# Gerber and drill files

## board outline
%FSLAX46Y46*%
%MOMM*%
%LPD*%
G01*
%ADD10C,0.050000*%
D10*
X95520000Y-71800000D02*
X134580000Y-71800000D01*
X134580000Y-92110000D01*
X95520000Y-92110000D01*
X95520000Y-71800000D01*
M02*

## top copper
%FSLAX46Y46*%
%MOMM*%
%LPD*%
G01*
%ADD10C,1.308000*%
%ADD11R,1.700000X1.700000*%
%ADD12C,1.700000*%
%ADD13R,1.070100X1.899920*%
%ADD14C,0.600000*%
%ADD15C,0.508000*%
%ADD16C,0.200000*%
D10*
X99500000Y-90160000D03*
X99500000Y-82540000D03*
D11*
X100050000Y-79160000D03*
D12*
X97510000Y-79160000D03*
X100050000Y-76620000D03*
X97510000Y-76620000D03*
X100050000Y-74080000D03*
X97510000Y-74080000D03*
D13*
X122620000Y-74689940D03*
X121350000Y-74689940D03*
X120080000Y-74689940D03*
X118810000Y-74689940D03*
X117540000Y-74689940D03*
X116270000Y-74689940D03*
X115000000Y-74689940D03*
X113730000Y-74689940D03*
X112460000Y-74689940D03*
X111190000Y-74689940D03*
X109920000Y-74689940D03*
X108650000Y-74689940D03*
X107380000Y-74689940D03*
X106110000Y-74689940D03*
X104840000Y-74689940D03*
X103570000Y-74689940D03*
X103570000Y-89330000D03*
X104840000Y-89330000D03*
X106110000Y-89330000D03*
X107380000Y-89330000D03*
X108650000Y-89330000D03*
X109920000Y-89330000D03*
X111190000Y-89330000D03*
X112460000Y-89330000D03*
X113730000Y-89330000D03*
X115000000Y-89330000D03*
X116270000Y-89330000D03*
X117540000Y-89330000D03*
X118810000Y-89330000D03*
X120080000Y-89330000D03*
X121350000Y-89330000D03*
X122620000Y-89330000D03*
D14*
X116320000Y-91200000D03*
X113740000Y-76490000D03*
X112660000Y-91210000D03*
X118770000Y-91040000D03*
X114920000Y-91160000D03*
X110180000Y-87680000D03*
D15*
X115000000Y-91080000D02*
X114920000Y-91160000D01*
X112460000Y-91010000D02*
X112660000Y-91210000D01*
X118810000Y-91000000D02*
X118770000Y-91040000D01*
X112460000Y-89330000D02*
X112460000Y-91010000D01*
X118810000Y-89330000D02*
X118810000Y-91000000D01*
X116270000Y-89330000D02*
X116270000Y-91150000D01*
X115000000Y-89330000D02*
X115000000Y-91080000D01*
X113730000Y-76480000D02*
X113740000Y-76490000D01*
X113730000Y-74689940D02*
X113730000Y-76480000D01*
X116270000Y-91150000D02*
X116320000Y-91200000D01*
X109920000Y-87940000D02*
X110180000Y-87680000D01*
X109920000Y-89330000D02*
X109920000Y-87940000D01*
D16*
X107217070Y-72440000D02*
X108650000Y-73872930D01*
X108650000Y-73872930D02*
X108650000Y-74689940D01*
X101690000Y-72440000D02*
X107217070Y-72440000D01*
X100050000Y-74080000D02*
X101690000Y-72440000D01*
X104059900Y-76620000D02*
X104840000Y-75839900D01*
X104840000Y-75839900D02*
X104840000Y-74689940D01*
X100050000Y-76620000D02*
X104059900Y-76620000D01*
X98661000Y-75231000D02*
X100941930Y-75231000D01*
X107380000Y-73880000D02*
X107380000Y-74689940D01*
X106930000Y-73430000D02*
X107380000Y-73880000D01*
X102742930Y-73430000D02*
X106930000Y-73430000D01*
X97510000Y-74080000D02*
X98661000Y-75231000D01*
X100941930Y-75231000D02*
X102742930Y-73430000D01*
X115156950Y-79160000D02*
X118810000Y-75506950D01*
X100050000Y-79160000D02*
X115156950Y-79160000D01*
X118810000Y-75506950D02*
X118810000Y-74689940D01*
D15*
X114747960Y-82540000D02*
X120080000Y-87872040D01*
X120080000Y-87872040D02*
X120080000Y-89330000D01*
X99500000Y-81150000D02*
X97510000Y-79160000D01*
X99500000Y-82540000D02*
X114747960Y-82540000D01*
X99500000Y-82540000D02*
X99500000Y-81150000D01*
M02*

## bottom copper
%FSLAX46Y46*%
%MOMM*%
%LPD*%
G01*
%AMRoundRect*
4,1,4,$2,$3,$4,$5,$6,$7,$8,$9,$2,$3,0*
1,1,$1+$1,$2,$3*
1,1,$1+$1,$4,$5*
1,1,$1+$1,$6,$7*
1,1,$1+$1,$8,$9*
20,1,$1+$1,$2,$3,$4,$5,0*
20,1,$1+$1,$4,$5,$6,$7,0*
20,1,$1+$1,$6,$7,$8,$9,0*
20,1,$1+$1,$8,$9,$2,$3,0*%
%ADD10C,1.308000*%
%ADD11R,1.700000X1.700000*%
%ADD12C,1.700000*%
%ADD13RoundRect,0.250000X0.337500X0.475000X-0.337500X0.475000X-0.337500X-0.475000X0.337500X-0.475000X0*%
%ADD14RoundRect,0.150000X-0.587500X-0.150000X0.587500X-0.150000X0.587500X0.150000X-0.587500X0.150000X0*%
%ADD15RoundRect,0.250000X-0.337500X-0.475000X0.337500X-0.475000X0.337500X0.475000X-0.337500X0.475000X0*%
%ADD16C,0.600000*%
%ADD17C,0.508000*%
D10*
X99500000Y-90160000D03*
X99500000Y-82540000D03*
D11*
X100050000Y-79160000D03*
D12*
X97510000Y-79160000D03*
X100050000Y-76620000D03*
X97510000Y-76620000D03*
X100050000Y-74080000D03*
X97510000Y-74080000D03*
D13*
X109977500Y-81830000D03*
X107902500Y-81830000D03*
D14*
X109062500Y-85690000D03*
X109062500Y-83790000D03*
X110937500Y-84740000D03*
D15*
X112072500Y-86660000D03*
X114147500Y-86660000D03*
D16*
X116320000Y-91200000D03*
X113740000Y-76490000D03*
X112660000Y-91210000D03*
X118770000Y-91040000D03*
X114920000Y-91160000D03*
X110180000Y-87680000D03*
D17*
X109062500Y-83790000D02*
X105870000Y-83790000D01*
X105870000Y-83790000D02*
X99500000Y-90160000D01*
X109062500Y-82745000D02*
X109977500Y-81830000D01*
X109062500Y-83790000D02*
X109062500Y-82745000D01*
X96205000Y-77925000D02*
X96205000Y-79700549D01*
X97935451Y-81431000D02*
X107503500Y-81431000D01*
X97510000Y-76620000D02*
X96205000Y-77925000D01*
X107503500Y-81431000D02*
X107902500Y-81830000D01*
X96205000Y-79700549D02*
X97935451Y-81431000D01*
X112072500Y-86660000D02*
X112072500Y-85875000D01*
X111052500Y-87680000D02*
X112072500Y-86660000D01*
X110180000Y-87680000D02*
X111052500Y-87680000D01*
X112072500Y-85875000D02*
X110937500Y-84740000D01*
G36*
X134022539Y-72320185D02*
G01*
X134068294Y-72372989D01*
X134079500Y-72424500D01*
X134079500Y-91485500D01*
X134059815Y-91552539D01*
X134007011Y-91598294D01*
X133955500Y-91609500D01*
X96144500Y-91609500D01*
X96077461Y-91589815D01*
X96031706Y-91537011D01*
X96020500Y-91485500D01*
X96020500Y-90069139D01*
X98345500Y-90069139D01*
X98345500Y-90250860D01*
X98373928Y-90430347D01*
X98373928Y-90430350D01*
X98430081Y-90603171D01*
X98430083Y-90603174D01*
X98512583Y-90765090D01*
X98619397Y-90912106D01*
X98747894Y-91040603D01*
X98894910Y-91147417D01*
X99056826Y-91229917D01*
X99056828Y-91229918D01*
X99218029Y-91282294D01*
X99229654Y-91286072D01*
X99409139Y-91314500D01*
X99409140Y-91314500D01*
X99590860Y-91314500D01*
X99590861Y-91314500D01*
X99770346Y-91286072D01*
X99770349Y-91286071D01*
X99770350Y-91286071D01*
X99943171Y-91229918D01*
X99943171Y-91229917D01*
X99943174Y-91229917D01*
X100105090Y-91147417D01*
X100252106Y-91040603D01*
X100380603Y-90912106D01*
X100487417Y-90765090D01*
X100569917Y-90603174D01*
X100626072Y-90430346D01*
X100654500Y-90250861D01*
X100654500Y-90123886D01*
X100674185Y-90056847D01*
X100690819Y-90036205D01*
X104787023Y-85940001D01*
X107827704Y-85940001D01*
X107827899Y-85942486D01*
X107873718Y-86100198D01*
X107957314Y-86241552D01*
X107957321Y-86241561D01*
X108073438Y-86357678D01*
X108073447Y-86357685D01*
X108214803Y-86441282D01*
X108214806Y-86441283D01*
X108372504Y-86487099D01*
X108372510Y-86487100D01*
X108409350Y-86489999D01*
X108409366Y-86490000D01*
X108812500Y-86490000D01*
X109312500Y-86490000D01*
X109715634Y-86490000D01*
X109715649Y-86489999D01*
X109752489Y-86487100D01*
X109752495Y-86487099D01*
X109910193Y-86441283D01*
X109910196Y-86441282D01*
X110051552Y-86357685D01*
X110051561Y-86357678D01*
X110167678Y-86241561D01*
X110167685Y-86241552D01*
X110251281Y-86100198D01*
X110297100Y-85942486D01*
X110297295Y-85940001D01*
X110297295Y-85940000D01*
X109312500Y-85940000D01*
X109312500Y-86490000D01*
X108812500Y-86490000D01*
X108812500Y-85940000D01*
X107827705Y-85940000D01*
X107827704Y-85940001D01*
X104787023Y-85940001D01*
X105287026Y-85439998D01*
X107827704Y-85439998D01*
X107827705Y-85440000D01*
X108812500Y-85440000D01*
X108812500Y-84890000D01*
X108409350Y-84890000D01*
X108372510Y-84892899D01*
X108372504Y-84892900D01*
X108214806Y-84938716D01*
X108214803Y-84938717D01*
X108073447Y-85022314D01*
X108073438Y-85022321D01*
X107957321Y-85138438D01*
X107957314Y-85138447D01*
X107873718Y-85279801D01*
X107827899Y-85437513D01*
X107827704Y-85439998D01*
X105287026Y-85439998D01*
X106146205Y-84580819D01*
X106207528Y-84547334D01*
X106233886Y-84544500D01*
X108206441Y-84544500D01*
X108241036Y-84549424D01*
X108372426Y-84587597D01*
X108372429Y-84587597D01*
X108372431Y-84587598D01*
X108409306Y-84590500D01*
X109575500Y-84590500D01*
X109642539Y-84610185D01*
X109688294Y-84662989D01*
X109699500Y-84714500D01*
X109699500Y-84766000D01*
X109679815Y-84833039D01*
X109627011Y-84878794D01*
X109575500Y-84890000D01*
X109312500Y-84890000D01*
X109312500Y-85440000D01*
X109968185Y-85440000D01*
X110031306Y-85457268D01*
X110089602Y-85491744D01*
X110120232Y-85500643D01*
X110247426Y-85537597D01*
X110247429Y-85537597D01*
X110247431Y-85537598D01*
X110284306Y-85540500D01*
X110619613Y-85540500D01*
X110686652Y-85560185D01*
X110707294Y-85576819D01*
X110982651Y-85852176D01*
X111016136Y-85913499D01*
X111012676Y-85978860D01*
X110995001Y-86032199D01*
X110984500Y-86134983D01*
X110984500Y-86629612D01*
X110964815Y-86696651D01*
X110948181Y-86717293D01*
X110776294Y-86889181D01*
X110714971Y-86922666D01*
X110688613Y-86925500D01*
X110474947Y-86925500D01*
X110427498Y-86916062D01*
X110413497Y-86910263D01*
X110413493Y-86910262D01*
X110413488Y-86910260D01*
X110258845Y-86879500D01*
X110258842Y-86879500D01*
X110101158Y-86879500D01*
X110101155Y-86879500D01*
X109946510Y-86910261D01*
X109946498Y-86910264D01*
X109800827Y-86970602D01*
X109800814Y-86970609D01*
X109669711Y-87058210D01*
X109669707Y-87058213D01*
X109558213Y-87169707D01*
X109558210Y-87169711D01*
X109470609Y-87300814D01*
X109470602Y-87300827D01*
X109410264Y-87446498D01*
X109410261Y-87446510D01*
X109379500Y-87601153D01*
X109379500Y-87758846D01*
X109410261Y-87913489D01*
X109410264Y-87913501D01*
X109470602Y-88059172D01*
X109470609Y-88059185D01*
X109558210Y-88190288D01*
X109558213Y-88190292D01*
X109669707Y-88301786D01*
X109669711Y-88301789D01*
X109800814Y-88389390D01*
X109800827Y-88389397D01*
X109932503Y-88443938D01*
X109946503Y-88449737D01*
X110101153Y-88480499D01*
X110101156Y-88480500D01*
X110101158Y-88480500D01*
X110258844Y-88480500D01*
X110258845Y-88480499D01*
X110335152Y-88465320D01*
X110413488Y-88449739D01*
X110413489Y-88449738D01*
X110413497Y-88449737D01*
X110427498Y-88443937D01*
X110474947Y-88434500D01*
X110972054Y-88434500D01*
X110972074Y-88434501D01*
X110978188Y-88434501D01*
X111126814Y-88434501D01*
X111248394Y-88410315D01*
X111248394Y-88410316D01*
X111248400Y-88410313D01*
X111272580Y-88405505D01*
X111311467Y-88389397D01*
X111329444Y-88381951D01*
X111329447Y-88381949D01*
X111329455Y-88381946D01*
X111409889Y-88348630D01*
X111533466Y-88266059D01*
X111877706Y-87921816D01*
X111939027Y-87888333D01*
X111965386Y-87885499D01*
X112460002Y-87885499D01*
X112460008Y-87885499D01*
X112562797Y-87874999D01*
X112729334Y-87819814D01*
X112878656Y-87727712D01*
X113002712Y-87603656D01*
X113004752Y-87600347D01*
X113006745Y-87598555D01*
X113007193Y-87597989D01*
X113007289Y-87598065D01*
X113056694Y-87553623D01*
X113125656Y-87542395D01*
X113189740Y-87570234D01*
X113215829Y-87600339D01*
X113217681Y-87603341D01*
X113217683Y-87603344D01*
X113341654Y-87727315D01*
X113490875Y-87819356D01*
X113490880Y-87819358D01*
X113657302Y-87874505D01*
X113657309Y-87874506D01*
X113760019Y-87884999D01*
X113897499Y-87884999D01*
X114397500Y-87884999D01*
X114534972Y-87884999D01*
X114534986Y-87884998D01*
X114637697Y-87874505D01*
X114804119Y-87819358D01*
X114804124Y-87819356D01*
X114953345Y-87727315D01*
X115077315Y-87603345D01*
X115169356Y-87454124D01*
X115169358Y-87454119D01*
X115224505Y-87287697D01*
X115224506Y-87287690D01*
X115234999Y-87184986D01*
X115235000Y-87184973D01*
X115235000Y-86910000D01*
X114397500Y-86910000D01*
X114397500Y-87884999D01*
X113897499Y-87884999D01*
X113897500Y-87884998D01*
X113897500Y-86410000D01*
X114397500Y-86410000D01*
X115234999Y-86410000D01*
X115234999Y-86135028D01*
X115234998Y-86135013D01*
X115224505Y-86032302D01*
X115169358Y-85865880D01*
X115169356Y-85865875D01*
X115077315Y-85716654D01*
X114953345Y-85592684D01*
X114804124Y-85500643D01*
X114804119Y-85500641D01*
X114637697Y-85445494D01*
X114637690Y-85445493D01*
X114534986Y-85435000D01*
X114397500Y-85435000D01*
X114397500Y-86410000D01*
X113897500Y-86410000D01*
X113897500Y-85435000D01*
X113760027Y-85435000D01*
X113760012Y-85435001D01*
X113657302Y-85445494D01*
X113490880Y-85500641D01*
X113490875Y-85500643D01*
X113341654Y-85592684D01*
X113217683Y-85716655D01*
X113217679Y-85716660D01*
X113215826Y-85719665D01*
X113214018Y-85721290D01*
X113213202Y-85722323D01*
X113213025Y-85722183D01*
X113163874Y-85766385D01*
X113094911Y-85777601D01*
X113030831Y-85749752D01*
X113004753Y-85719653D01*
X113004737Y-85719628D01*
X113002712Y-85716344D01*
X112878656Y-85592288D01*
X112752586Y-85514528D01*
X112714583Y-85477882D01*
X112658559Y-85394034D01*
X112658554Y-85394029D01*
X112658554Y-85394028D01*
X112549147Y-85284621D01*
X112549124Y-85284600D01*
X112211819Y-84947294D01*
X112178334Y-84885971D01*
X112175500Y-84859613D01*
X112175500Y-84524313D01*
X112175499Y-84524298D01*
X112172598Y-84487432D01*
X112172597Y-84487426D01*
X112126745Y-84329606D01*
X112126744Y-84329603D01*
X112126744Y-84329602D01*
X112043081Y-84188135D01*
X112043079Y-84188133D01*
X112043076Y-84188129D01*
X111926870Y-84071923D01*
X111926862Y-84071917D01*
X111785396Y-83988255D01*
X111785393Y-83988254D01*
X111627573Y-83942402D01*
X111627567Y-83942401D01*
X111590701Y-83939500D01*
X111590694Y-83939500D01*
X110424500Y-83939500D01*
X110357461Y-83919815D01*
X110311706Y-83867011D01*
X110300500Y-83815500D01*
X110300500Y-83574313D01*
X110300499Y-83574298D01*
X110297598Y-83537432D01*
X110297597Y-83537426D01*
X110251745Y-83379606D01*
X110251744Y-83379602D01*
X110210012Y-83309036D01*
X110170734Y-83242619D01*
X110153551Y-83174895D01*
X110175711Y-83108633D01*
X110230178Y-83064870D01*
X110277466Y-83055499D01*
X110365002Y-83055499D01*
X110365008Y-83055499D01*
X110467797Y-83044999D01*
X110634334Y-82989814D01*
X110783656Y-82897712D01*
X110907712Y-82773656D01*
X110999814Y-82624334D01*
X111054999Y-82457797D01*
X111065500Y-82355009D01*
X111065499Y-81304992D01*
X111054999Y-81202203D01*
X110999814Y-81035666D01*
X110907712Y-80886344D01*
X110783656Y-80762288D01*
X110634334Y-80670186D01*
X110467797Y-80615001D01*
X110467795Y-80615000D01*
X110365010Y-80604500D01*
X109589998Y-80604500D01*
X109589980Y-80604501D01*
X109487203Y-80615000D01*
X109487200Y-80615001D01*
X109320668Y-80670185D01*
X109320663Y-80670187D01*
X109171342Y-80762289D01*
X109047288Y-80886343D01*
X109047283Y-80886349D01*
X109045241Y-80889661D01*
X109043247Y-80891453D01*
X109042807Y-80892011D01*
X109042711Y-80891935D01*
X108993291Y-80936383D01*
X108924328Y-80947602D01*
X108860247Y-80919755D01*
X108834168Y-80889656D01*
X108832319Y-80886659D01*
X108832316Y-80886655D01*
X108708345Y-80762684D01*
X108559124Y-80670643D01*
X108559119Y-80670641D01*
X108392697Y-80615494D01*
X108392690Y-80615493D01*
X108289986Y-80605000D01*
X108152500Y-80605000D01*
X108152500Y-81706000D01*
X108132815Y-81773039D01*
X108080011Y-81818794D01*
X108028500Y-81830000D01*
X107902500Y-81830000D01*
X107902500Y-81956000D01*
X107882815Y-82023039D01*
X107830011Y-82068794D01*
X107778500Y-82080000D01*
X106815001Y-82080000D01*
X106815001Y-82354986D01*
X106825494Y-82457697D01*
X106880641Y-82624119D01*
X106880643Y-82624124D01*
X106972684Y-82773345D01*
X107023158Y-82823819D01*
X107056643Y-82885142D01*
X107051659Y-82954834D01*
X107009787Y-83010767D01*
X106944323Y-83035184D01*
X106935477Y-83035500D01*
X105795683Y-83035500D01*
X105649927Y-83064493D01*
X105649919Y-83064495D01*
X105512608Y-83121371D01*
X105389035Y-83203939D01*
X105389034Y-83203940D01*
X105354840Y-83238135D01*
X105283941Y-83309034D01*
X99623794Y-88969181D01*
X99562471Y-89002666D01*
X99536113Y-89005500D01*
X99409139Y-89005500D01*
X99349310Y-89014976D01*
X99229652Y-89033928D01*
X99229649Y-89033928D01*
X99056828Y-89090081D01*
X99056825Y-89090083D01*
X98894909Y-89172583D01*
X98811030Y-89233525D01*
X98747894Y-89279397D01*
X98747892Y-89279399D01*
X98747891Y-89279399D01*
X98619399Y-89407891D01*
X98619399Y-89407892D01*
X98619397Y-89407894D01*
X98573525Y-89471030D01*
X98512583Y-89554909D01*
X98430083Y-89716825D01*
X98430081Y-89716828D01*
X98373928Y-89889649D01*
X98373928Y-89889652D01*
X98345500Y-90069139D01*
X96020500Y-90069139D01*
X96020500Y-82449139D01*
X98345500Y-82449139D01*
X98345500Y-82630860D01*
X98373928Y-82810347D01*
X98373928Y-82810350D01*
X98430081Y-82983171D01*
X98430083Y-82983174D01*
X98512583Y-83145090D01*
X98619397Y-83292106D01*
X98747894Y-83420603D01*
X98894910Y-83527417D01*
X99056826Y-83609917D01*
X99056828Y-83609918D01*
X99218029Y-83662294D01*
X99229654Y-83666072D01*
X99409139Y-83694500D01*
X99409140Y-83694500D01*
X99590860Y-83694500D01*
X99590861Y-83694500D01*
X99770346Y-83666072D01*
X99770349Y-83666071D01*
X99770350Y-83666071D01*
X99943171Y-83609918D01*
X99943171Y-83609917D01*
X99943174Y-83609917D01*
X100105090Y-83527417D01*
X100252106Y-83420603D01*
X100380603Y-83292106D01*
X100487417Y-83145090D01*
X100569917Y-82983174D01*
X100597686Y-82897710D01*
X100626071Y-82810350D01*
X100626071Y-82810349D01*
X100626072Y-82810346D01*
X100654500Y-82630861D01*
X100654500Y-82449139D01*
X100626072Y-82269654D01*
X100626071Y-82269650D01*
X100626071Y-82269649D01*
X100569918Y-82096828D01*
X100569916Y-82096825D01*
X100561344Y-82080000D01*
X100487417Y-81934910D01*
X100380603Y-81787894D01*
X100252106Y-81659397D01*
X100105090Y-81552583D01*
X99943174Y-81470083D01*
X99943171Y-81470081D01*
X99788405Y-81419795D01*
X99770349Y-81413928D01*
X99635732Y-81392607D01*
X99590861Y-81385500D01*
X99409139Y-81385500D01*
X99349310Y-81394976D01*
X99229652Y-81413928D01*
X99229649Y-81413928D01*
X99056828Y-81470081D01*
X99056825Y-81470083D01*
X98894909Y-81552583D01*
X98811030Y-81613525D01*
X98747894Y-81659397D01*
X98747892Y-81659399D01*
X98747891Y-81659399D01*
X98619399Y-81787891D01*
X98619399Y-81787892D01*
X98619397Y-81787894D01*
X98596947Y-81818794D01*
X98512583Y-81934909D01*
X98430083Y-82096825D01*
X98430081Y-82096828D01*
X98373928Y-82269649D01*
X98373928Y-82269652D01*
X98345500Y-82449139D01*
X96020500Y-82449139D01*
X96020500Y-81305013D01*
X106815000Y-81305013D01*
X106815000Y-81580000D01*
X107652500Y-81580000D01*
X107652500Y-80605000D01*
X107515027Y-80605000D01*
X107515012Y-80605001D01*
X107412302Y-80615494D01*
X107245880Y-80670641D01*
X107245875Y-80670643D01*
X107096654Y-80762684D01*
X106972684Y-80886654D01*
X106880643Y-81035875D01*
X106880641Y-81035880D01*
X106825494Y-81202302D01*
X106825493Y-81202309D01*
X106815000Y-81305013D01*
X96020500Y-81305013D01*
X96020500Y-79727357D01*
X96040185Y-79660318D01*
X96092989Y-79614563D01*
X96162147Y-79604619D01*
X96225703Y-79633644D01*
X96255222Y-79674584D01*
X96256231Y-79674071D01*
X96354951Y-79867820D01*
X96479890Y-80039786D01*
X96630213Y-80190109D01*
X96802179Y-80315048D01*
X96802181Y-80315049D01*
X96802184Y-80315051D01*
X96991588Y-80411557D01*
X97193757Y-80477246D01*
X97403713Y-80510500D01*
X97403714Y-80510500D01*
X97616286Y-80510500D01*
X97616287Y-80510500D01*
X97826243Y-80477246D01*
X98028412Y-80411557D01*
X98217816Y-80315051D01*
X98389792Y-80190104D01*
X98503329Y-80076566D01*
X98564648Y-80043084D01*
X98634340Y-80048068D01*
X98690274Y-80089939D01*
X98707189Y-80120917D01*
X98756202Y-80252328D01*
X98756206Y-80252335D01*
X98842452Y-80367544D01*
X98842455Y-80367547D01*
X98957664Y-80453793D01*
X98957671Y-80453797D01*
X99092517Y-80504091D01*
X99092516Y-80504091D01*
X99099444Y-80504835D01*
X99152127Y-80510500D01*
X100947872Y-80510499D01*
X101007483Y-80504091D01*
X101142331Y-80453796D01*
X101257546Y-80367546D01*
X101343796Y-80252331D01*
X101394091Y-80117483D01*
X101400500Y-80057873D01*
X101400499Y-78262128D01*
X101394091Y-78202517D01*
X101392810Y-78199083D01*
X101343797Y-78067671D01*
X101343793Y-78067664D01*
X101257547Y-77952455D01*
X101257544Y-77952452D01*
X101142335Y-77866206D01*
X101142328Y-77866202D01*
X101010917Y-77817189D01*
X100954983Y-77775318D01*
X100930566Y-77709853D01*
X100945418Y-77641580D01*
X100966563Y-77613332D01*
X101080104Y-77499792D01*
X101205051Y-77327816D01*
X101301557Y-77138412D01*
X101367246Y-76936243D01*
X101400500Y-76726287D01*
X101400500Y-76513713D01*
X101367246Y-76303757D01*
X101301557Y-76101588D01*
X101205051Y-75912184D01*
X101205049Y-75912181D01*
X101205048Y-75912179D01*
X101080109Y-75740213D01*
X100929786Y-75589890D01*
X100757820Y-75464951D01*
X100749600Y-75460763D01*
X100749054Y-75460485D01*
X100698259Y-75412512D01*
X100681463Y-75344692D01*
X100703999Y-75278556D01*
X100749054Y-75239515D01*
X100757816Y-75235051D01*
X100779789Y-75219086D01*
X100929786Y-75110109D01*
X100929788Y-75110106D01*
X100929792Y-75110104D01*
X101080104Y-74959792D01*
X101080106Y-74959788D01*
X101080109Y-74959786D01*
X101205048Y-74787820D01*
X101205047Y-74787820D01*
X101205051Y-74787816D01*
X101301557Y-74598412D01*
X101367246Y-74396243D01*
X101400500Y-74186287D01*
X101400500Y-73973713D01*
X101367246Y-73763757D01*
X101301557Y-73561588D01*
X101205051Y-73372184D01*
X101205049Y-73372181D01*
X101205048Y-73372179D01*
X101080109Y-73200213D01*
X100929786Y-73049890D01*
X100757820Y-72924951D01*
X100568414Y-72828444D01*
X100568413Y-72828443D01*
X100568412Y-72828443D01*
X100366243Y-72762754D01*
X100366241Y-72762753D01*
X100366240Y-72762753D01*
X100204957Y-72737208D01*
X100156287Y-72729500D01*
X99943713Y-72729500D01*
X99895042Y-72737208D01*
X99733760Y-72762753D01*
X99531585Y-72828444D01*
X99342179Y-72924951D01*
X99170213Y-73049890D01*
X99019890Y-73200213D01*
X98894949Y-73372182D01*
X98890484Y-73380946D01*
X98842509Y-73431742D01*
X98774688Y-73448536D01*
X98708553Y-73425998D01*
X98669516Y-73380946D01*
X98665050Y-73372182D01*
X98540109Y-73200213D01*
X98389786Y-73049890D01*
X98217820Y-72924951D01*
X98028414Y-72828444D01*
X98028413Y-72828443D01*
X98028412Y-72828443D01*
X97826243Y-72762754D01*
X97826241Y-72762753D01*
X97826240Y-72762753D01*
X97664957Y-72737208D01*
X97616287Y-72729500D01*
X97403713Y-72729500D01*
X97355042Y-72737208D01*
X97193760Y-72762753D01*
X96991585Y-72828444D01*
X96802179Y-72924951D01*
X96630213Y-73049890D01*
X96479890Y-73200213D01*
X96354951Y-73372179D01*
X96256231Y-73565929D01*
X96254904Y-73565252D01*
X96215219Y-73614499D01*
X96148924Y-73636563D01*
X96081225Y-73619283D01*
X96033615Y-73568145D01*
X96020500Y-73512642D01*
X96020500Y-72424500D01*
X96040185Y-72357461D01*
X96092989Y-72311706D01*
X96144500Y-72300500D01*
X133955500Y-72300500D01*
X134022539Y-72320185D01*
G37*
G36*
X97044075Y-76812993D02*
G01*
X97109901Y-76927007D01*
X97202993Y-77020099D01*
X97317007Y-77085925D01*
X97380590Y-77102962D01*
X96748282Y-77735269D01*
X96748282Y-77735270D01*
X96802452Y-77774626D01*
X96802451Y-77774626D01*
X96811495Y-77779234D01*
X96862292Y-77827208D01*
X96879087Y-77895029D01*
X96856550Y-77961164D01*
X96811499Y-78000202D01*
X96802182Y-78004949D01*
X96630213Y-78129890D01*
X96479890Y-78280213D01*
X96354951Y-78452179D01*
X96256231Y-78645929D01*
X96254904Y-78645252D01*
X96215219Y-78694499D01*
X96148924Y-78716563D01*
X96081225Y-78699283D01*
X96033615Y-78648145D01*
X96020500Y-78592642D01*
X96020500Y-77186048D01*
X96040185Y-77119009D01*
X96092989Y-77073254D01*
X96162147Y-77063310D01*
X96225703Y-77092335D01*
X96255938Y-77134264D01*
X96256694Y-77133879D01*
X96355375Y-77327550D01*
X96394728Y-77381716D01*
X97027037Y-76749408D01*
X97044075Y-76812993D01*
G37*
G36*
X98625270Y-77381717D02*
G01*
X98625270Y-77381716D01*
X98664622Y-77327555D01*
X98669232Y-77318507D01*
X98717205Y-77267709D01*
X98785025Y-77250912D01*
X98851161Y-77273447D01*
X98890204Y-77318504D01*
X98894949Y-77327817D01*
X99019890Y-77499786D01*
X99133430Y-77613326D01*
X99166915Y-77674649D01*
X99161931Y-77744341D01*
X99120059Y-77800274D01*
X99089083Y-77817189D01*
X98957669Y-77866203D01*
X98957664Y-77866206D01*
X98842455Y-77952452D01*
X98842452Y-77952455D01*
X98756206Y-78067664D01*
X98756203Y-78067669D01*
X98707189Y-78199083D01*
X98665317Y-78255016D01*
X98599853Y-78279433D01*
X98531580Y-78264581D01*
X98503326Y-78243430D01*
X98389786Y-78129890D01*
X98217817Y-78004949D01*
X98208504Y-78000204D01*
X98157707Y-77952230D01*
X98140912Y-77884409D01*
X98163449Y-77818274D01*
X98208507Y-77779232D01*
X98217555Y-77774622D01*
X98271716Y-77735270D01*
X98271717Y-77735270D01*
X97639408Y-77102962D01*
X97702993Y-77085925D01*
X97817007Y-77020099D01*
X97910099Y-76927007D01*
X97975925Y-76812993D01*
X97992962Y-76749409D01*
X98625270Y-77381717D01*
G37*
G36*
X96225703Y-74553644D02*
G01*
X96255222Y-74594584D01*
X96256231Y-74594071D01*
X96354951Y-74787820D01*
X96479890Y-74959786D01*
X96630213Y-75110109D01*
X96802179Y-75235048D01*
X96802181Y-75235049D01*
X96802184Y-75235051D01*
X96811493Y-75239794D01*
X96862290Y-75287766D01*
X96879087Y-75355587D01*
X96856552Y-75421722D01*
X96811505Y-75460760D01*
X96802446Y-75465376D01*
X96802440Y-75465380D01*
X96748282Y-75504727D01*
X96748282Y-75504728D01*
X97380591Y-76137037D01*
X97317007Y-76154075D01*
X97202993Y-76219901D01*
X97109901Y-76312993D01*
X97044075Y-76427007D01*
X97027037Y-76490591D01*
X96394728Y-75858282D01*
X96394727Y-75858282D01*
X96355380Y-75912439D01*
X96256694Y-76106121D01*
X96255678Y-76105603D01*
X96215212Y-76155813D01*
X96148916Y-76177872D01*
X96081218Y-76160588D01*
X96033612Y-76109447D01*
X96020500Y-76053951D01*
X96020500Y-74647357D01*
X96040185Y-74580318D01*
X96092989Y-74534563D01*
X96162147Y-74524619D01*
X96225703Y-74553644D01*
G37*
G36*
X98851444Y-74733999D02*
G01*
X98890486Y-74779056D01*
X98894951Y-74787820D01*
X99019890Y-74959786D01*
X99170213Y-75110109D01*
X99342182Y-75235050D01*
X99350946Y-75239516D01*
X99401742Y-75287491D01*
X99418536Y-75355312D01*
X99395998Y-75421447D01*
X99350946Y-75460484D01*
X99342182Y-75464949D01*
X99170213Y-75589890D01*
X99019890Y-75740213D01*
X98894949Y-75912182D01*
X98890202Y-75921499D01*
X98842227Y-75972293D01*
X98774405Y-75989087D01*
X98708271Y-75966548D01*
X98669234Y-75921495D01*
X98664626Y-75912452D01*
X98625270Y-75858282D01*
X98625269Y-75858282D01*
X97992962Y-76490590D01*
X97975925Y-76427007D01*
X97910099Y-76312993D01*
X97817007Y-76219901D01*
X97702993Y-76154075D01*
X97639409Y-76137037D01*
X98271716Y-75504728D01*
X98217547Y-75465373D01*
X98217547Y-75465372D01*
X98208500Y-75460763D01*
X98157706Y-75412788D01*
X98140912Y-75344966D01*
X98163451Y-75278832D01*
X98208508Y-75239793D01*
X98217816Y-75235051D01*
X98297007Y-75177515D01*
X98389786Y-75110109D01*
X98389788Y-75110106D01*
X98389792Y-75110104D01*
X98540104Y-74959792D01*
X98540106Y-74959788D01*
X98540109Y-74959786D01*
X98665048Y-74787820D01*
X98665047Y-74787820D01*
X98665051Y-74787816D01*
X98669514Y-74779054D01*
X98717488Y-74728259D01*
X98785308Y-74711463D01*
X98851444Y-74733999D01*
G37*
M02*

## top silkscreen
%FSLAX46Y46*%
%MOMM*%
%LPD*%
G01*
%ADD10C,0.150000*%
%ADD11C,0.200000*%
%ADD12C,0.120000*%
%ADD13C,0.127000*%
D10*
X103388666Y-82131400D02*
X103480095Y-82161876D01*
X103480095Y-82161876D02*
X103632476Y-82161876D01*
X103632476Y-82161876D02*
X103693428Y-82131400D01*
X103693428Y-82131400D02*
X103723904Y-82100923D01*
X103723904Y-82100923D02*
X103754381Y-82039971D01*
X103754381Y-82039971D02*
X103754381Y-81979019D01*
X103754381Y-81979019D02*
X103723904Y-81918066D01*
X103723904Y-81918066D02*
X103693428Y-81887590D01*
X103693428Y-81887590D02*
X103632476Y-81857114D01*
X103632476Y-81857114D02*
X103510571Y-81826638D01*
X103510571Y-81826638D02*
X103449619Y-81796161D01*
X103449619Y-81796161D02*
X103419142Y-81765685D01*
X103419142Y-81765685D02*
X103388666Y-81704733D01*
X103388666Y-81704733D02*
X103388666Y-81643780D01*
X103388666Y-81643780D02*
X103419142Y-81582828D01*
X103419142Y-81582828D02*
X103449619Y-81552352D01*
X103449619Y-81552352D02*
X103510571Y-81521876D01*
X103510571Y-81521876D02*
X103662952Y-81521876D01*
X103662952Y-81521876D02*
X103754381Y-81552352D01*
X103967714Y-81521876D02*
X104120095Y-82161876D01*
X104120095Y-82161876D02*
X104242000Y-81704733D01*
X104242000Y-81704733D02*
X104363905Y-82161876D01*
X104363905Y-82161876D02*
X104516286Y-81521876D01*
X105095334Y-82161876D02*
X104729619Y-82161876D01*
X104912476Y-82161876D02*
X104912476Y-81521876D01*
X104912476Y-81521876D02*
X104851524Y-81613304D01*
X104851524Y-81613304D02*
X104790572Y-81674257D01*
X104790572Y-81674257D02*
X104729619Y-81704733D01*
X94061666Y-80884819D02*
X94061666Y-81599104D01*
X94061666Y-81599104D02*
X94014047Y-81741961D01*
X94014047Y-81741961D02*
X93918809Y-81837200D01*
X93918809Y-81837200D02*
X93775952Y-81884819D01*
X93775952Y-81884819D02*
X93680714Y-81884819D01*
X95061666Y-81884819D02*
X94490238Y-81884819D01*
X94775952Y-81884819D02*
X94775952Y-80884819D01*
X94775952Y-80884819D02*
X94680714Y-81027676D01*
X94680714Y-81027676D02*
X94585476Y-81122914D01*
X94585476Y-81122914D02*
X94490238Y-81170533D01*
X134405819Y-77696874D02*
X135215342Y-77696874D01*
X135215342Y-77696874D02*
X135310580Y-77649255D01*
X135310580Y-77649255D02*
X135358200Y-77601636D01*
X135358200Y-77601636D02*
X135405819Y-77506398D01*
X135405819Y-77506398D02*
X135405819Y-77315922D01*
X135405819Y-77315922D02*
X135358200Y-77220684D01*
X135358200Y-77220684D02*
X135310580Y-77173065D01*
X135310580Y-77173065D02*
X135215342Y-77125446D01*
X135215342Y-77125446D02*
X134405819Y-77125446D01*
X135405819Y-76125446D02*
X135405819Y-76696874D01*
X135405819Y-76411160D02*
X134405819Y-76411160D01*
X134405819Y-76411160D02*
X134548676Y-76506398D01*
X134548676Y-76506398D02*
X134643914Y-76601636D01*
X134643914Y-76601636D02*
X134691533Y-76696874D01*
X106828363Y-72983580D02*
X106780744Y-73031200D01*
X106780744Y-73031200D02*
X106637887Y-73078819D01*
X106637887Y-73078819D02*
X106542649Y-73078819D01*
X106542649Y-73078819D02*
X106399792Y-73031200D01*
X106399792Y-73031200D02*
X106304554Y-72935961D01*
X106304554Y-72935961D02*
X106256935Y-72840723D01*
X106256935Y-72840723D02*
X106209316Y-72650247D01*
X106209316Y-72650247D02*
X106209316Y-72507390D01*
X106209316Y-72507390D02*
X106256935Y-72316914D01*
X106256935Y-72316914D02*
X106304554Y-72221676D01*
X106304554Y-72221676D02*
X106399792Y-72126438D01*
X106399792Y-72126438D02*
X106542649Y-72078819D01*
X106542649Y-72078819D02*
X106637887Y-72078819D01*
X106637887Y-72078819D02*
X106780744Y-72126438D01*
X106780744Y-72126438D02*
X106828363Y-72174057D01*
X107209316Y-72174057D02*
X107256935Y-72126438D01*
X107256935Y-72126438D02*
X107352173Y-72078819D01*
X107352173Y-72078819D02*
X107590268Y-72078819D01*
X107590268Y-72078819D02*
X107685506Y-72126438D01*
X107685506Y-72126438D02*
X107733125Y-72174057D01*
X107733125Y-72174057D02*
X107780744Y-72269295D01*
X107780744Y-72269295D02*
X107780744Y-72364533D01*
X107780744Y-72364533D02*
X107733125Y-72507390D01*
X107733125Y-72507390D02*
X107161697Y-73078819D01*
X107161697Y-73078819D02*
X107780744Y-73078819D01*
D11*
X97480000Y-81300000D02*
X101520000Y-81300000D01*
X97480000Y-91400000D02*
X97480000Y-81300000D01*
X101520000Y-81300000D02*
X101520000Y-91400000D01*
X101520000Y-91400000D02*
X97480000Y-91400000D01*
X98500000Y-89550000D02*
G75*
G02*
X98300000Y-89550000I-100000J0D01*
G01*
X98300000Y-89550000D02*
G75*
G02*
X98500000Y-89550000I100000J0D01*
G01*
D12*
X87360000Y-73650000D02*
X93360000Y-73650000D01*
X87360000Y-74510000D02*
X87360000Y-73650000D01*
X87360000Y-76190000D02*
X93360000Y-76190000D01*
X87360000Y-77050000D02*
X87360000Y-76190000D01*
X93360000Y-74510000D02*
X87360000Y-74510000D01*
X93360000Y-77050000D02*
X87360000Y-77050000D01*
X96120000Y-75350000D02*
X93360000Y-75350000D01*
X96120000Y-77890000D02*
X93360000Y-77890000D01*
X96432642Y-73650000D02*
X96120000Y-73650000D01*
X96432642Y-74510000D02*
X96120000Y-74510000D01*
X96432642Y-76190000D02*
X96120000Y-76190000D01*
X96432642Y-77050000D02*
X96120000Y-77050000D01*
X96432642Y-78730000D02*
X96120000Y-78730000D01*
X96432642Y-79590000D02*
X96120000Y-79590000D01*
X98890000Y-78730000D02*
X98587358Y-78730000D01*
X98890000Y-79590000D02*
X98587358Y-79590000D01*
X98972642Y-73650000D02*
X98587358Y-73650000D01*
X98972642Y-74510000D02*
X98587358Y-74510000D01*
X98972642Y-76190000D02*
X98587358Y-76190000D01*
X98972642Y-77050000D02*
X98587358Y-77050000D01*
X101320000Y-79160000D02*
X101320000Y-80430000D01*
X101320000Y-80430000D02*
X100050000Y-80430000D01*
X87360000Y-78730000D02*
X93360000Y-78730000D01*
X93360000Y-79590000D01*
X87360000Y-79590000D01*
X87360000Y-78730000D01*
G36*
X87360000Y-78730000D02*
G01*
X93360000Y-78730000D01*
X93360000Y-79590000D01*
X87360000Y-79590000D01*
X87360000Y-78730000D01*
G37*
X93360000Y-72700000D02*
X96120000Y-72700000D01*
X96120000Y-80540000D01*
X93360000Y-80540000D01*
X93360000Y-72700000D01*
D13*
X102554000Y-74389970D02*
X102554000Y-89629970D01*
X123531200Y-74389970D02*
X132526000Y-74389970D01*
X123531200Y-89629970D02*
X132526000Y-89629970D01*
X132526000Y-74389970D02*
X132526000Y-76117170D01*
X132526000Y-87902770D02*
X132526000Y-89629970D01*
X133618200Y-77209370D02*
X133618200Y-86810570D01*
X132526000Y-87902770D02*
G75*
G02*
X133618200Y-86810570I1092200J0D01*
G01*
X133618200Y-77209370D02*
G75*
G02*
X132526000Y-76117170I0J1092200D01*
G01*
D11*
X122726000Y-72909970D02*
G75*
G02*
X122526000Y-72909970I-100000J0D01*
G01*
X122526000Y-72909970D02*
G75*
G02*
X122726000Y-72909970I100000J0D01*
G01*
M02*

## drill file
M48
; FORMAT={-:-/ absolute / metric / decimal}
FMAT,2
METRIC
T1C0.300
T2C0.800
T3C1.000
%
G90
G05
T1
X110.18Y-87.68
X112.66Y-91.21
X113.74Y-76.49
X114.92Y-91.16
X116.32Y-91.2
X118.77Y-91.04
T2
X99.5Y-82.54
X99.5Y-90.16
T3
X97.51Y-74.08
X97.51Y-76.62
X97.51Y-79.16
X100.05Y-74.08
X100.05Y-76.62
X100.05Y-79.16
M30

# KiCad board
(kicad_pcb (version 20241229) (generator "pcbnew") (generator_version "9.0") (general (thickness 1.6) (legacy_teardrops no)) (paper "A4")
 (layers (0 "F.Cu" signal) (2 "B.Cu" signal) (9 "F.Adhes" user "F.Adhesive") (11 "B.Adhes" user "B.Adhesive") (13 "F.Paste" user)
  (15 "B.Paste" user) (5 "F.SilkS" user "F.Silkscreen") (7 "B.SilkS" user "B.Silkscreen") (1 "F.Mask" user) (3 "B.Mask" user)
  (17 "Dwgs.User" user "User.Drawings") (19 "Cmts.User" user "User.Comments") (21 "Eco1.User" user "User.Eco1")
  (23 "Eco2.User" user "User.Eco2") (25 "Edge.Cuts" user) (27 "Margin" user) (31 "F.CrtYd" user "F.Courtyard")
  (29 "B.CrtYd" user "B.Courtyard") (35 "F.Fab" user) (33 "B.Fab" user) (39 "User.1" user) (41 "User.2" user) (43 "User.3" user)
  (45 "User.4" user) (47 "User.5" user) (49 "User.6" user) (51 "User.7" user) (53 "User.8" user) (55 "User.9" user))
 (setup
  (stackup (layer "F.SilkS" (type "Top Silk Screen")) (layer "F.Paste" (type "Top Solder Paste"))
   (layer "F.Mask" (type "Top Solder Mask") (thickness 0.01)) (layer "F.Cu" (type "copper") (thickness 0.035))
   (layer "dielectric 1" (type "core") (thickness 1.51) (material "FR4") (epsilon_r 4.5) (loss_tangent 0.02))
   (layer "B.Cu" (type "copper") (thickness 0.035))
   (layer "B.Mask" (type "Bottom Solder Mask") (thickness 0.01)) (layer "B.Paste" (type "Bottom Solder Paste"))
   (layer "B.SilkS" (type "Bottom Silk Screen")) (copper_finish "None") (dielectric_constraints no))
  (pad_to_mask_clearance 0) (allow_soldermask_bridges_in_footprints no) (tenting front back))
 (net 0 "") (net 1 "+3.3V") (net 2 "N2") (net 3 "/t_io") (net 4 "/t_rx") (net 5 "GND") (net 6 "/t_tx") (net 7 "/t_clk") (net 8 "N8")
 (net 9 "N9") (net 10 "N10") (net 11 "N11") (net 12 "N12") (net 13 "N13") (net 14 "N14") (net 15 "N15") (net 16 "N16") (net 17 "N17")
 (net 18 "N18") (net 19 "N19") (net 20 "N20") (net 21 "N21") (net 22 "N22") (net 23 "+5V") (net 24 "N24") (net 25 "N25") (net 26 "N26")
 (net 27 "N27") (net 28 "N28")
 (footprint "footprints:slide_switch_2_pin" (layer "F.Cu") (at 99.5 86.35)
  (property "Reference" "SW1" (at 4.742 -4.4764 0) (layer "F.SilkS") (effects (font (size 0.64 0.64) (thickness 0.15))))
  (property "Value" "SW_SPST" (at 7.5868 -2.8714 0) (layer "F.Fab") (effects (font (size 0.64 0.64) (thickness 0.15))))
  (fp_line (start -2.02 -5.05) (end 2.02 -5.05) (stroke (width 0.2) (type solid)) (layer "F.SilkS"))
  (fp_line (start -2.02 5.05) (end -2.02 -5.05) (stroke (width 0.2) (type solid)) (layer "F.SilkS"))
  (fp_line (start 2.02 -5.05) (end 2.02 5.05) (stroke (width 0.2) (type solid)) (layer "F.SilkS"))
  (fp_line (start 2.02 5.05) (end -2.02 5.05) (stroke (width 0.2) (type solid)) (layer "F.SilkS"))
  (fp_circle (center -1.1 3.2) (end -1 3.2) (stroke (width 0.2) (type solid)) (fill no) (layer "F.SilkS"))
  (pad "1" thru_hole circle (at 0 3.81) (size 1.308 1.308) (drill 0.8) (layers "*.Cu" "*.Mask") (remove_unused_layers no) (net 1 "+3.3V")
   (solder_mask_margin 0.102))
  (pad "2" thru_hole circle (at 0 -3.81) (size 1.308 1.308) (drill 0.8) (layers "*.Cu" "*.Mask") (remove_unused_layers no) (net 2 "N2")
   (solder_mask_margin 0.102)))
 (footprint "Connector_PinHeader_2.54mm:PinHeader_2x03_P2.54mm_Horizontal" (layer "F.Cu") (at 100.05 79.16 180)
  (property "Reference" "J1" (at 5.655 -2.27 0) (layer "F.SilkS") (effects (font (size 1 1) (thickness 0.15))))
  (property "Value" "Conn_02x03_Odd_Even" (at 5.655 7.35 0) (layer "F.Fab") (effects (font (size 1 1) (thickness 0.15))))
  (fp_line (start 12.69 5.51) (end 6.69 5.51) (stroke (width 0.12) (type solid)) (layer "F.SilkS"))
  (fp_line (start 12.69 4.65) (end 12.69 5.51) (stroke (width 0.12) (type solid)) (layer "F.SilkS"))
  (fp_line (start 12.69 2.97) (end 6.69 2.97) (stroke (width 0.12) (type solid)) (layer "F.SilkS"))
  (fp_line (start 12.69 2.11) (end 12.69 2.97) (stroke (width 0.12) (type solid)) (layer "F.SilkS"))
  (fp_line (start 6.69 4.65) (end 12.69 4.65) (stroke (width 0.12) (type solid)) (layer "F.SilkS"))
  (fp_line (start 6.69 2.11) (end 12.69 2.11) (stroke (width 0.12) (type solid)) (layer "F.SilkS"))
  (fp_line (start 3.93 3.81) (end 6.69 3.81) (stroke (width 0.12) (type solid)) (layer "F.SilkS"))
  (fp_line (start 3.93 1.27) (end 6.69 1.27) (stroke (width 0.12) (type solid)) (layer "F.SilkS"))
  (fp_line (start 3.617358 5.51) (end 3.93 5.51) (stroke (width 0.12) (type solid)) (layer "F.SilkS"))
  (fp_line (start 3.617358 4.65) (end 3.93 4.65) (stroke (width 0.12) (type solid)) (layer "F.SilkS"))
  (fp_line (start 3.617358 2.97) (end 3.93 2.97) (stroke (width 0.12) (type solid)) (layer "F.SilkS"))
  (fp_line (start 3.617358 2.11) (end 3.93 2.11) (stroke (width 0.12) (type solid)) (layer "F.SilkS"))
  (fp_line (start 3.617358 0.43) (end 3.93 0.43) (stroke (width 0.12) (type solid)) (layer "F.SilkS"))
  (fp_line (start 3.617358 -0.43) (end 3.93 -0.43) (stroke (width 0.12) (type solid)) (layer "F.SilkS"))
  (fp_line (start 1.16 0.43) (end 1.462642 0.43) (stroke (width 0.12) (type solid)) (layer "F.SilkS"))
  (fp_line (start 1.16 -0.43) (end 1.462642 -0.43) (stroke (width 0.12) (type solid)) (layer "F.SilkS"))
  (fp_line (start 1.077358 5.51) (end 1.462642 5.51) (stroke (width 0.12) (type solid)) (layer "F.SilkS"))
  (fp_line (start 1.077358 4.65) (end 1.462642 4.65) (stroke (width 0.12) (type solid)) (layer "F.SilkS"))
  (fp_line (start 1.077358 2.97) (end 1.462642 2.97) (stroke (width 0.12) (type solid)) (layer "F.SilkS"))
  (fp_line (start 1.077358 2.11) (end 1.462642 2.11) (stroke (width 0.12) (type solid)) (layer "F.SilkS"))
  (fp_line (start -1.27 0) (end -1.27 -1.27) (stroke (width 0.12) (type solid)) (layer "F.SilkS"))
  (fp_line (start -1.27 -1.27) (end 0 -1.27) (stroke (width 0.12) (type solid)) (layer "F.SilkS"))
  (fp_rect (start 6.69 -0.43) (end 12.69 0.43) (stroke (width 0.12) (type solid)) (fill yes) (layer "F.SilkS"))
  (fp_rect (start 3.93 -1.38) (end 6.69 6.46) (stroke (width 0.12) (type solid)) (fill no) (layer "F.SilkS"))
  (pad "1" thru_hole rect (at 0 0 180) (size 1.7 1.7) (drill 1) (layers "*.Cu" "*.Mask") (remove_unused_layers no) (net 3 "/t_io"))
  (pad "2" thru_hole circle (at 2.54 0 180) (size 1.7 1.7) (drill 1) (layers "*.Cu" "*.Mask") (remove_unused_layers no) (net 2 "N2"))
  (pad "3" thru_hole circle (at 0 2.54 180) (size 1.7 1.7) (drill 1) (layers "*.Cu" "*.Mask") (remove_unused_layers no) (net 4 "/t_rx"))
  (pad "4" thru_hole circle (at 2.54 2.54 180) (size 1.7 1.7) (drill 1) (layers "*.Cu" "*.Mask") (remove_unused_layers no) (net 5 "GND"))
  (pad "5" thru_hole circle (at 0 5.08 180) (size 1.7 1.7) (drill 1) (layers "*.Cu" "*.Mask") (remove_unused_layers no) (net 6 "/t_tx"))
  (pad "6" thru_hole circle (at 2.54 5.08 180) (size 1.7 1.7) (drill 1) (layers "*.Cu" "*.Mask") (remove_unused_layers no) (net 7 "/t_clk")))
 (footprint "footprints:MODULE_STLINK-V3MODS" (layer "F.Cu") (at 132.526 82.00997 -90)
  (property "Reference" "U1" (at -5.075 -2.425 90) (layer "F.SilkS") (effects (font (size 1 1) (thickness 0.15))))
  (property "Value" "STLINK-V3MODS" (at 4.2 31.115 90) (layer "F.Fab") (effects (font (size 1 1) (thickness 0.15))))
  (fp_line (start -7.62 29.972) (end 7.62 29.972) (stroke (width 0.127) (type solid)) (layer "F.SilkS"))
  (fp_line (start -7.62 8.9948) (end -7.62 0) (stroke (width 0.127) (type solid)) (layer "F.SilkS"))
  (fp_line (start 7.62 8.9948) (end 7.62 0) (stroke (width 0.127) (type solid)) (layer "F.SilkS"))
  (fp_line (start -7.62 0) (end -5.8928 0) (stroke (width 0.127) (type solid)) (layer "F.SilkS"))
  (fp_line (start 5.8928 0) (end 7.62 0) (stroke (width 0.127) (type solid)) (layer "F.SilkS"))
  (fp_line (start -4.8006 -1.0922) (end 4.8006 -1.0922) (stroke (width 0.127) (type solid)) (layer "F.SilkS"))
  (fp_arc (start 5.8928 0) (mid 5.120498 -0.319898) (end 4.8006 -1.0922) (stroke (width 0.127) (type solid)) (layer "F.SilkS"))
  (fp_arc (start -4.8006 -1.0922) (mid -5.120498 -0.319898) (end -5.8928 0) (stroke (width 0.127) (type solid)) (layer "F.SilkS"))
  (fp_circle (center -9.1 9.9) (end -9 9.9) (stroke (width 0.2) (type solid)) (fill no) (layer "F.SilkS"))
  (pad "1" smd rect (at -7.32003 9.906 270) (size 1.89992 1.0701) (layers "F.Cu" "F.Mask" "F.Paste") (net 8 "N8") (solder_mask_margin 0.102))
  (pad "2" smd rect (at -7.32003 11.176 270) (size 1.89992 1.0701) (layers "F.Cu" "F.Mask" "F.Paste") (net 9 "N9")
   (solder_mask_margin 0.102))
  (pad "3" smd rect (at -7.32003 12.446 270) (size 1.89992 1.0701) (layers "F.Cu" "F.Mask" "F.Paste") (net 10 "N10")
   (solder_mask_margin 0.102))
  (pad "4" smd rect (at -7.32003 13.716 270) (size 1.89992 1.0701) (layers "F.Cu" "F.Mask" "F.Paste") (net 3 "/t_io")
   (solder_mask_margin 0.102))
  (pad "5" smd rect (at -7.32003 14.986 270) (size 1.89992 1.0701) (layers "F.Cu" "F.Mask" "F.Paste") (solder_mask_margin 0.102))
  (pad "6" smd rect (at -7.32003 16.256 270) (size 1.89992 1.0701) (layers "F.Cu" "F.Mask" "F.Paste") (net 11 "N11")
   (solder_mask_margin 0.102))
  (pad "7" smd rect (at -7.32003 17.526 270) (size 1.89992 1.0701) (layers "F.Cu" "F.Mask" "F.Paste") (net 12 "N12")
   (solder_mask_margin 0.102))
  (pad "8" smd rect (at -7.32003 18.796 270) (size 1.89992 1.0701) (layers "F.Cu" "F.Mask" "F.Paste") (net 5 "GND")
   (solder_mask_margin 0.102))
  (pad "9" smd rect (at -7.32003 20.066 270) (size 1.89992 1.0701) (layers "F.Cu" "F.Mask" "F.Paste") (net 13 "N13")
   (solder_mask_margin 0.102))
  (pad "10" smd rect (at -7.32003 21.336 270) (size 1.89992 1.0701) (layers "F.Cu" "F.Mask" "F.Paste") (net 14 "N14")
   (solder_mask_margin 0.102))
  (pad "11" smd rect (at -7.32003 22.606 270) (size 1.89992 1.0701) (layers "F.Cu" "F.Mask" "F.Paste") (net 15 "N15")
   (solder_mask_margin 0.102))
  (pad "12" smd rect (at -7.32003 23.876 270) (size 1.89992 1.0701) (layers "F.Cu" "F.Mask" "F.Paste") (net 6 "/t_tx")
   (solder_mask_margin 0.102))
  (pad "13" smd rect (at -7.32003 25.146 270) (size 1.89992 1.0701) (layers "F.Cu" "F.Mask" "F.Paste") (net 7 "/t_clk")
   (solder_mask_margin 0.102))
  (pad "14" smd rect (at -7.32003 26.416 270) (size 1.89992 1.0701) (layers "F.Cu" "F.Mask" "F.Paste") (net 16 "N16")
   (solder_mask_margin 0.102))
  (pad "15" smd rect (at -7.32003 27.686 270) (size 1.89992 1.0701) (layers "F.Cu" "F.Mask" "F.Paste") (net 4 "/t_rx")
   (solder_mask_margin 0.102))
  (pad "16" smd rect (at -7.32003 28.956 270) (size 1.89992 1.0701) (layers "F.Cu" "F.Mask" "F.Paste") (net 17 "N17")
   (solder_mask_margin 0.102))
  (pad "17" smd rect (at 7.32003 28.956 270) (size 1.89992 1.0701) (layers "F.Cu" "F.Mask" "F.Paste") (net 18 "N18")
   (solder_mask_margin 0.102))
  (pad "18" smd rect (at 7.32003 27.686 270) (size 1.89992 1.0701) (layers "F.Cu" "F.Mask" "F.Paste") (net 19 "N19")
   (solder_mask_margin 0.102))
  (pad "19" smd rect (at 7.32003 26.416 270) (size 1.89992 1.0701) (layers "F.Cu" "F.Mask" "F.Paste") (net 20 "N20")
   (solder_mask_margin 0.102))
  (pad "20" smd rect (at 7.32003 25.146 270) (size 1.89992 1.0701) (layers "F.Cu" "F.Mask" "F.Paste") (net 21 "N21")
   (solder_mask_margin 0.102))
  (pad "21" smd rect (at 7.32003 23.876 270) (size 1.89992 1.0701) (layers "F.Cu" "F.Mask" "F.Paste") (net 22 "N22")
   (solder_mask_margin 0.102))
  (pad "22" smd rect (at 7.32003 22.606 270) (size 1.89992 1.0701) (layers "F.Cu" "F.Mask" "F.Paste") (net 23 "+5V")
   (solder_mask_margin 0.102))
  (pad "23" smd rect (at 7.32003 21.336 270) (size 1.89992 1.0701) (layers "F.Cu" "F.Mask" "F.Paste") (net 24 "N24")
   (solder_mask_margin 0.102))
  (pad "24" smd rect (at 7.32003 20.066 270) (size 1.89992 1.0701) (layers "F.Cu" "F.Mask" "F.Paste") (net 5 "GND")
   (solder_mask_margin 0.102))
  (pad "25" smd rect (at 7.32003 18.796 270) (size 1.89992 1.0701) (layers "F.Cu" "F.Mask" "F.Paste") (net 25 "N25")
   (solder_mask_margin 0.102))
  (pad "26" smd rect (at 7.32003 17.526 270) (size 1.89992 1.0701) (layers "F.Cu" "F.Mask" "F.Paste") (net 5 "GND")
   (solder_mask_margin 0.102))
  (pad "27" smd rect (at 7.32003 16.256 270) (size 1.89992 1.0701) (layers "F.Cu" "F.Mask" "F.Paste") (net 5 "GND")
   (solder_mask_margin 0.102))
  (pad "28" smd rect (at 7.32003 14.986 270) (size 1.89992 1.0701) (layers "F.Cu" "F.Mask" "F.Paste") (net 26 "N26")
   (solder_mask_margin 0.102))
  (pad "29" smd rect (at 7.32003 13.716 270) (size 1.89992 1.0701) (layers "F.Cu" "F.Mask" "F.Paste") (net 5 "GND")
   (solder_mask_margin 0.102))
  (pad "30" smd rect (at 7.32003 12.446 270) (size 1.89992 1.0701) (layers "F.Cu" "F.Mask" "F.Paste") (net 2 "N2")
   (solder_mask_margin 0.102))
  (pad "31" smd rect (at 7.32003 11.176 270) (size 1.89992 1.0701) (layers "F.Cu" "F.Mask" "F.Paste") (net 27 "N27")
   (solder_mask_margin 0.102))
  (pad "32" smd rect (at 7.32003 9.906 270) (size 1.89992 1.0701) (layers "F.Cu" "F.Mask" "F.Paste") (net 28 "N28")
   (solder_mask_margin 0.102)))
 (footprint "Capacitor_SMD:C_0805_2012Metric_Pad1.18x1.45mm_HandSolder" (layer "B.Cu") (at 108.94 81.83 180)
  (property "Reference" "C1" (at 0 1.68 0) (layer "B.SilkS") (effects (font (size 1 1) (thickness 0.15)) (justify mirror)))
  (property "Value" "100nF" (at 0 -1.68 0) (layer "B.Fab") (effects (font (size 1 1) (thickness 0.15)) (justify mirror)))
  (pad "1" smd roundrect (at -1.0375 0 180) (size 1.175 1.45) (layers "B.Cu" "B.Mask" "B.Paste") (roundrect_rratio 0.212766) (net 1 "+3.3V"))
  (pad "2" smd roundrect (at 1.0375 0 180) (size 1.175 1.45) (layers "B.Cu" "B.Mask" "B.Paste") (roundrect_rratio 0.212766) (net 5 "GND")))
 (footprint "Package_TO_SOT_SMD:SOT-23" (layer "B.Cu") (at 110 84.74)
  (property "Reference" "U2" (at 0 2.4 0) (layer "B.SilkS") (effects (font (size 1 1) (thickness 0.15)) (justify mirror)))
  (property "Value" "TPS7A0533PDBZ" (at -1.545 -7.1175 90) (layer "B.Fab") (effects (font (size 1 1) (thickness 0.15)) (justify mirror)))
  (pad "1" smd roundrect (at -0.9375 0.95) (size 1.475 0.6) (layers "B.Cu" "B.Mask" "B.Paste") (roundrect_rratio 0.25) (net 5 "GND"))
  (pad "2" smd roundrect (at -0.9375 -0.95) (size 1.475 0.6) (layers "B.Cu" "B.Mask" "B.Paste") (roundrect_rratio 0.25) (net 1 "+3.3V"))
  (pad "3" smd roundrect (at 0.9375 0) (size 1.475 0.6) (layers "B.Cu" "B.Mask" "B.Paste") (roundrect_rratio 0.25) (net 23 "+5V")))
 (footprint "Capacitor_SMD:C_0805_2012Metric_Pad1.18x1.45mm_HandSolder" (layer "B.Cu") (at 113.11 86.66)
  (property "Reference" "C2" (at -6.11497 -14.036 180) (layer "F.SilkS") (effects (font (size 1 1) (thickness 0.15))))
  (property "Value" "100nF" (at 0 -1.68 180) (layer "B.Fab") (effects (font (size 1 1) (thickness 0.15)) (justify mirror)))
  (pad "1" smd roundrect (at -1.0375 0) (size 1.175 1.45) (layers "B.Cu" "B.Mask" "B.Paste") (roundrect_rratio 0.212766) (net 23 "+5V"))
  (pad "2" smd roundrect (at 1.0375 0) (size 1.175 1.45) (layers "B.Cu" "B.Mask" "B.Paste") (roundrect_rratio 0.212766) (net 5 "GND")))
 (gr_rect (start 95.52 71.8) (end 134.58 92.11) (stroke (width 0.05) (type default)) (fill no) (layer "Edge.Cuts"))
 (segment (start 109.0625 83.79) (end 105.87 83.79) (width 0.508) (layer "B.Cu") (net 1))
 (segment (start 105.87 83.79) (end 99.5 90.16) (width 0.508) (layer "B.Cu") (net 1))
 (segment (start 109.0625 82.745) (end 109.9775 81.83) (width 0.508) (layer "B.Cu") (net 1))
 (segment (start 109.0625 83.79) (end 109.0625 82.745) (width 0.508) (layer "B.Cu") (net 1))
 (segment (start 115 91.08) (end 114.92 91.16) (width 0.508) (layer "F.Cu") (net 5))
 (segment (start 112.46 91.01) (end 112.66 91.21) (width 0.508) (layer "F.Cu") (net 5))
 (segment (start 118.81 91) (end 118.77 91.04) (width 0.508) (layer "F.Cu") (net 5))
 (segment (start 112.46 89.33) (end 112.46 91.01) (width 0.508) (layer "F.Cu") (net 5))
 (segment (start 118.81 89.33) (end 118.81 91) (width 0.508) (layer "F.Cu") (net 5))
 (segment (start 116.27 89.33) (end 116.27 91.15) (width 0.508) (layer "F.Cu") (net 5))
 (segment (start 115 89.33) (end 115 91.08) (width 0.508) (layer "F.Cu") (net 5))
 (segment (start 113.73 76.48) (end 113.74 76.49) (width 0.508) (layer "F.Cu") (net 5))
 (segment (start 113.73 74.68994) (end 113.73 76.48) (width 0.508) (layer "F.Cu") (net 5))
 (segment (start 116.27 91.15) (end 116.32 91.2) (width 0.508) (layer "F.Cu") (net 5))
 (via (at 116.32 91.2) (size 0.6) (drill 0.3) (layers "F.Cu" "B.Cu") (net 5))
 (via (at 113.74 76.49) (size 0.6) (drill 0.3) (layers "F.Cu" "B.Cu") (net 5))
 (via (at 112.66 91.21) (size 0.6) (drill 0.3) (layers "F.Cu" "B.Cu") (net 5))
 (via (at 118.77 91.04) (size 0.6) (drill 0.3) (layers "F.Cu" "B.Cu") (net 5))
 (via (at 114.92 91.16) (size 0.6) (drill 0.3) (layers "F.Cu" "B.Cu") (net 5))
 (segment (start 96.205 77.925) (end 96.205 79.700549) (width 0.508) (layer "B.Cu") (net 5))
 (segment (start 97.935451 81.431) (end 107.5035 81.431) (width 0.508) (layer "B.Cu") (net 5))
 (segment (start 97.51 76.62) (end 96.205 77.925) (width 0.508) (layer "B.Cu") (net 5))
 (segment (start 107.5035 81.431) (end 107.9025 81.83) (width 0.508) (layer "B.Cu") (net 5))
 (segment (start 96.205 79.700549) (end 97.935451 81.431) (width 0.508) (layer "B.Cu") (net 5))
 (segment (start 109.92 87.94) (end 110.18 87.68) (width 0.508) (layer "F.Cu") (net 23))
 (segment (start 109.92 89.33) (end 109.92 87.94) (width 0.508) (layer "F.Cu") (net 23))
 (via (at 110.18 87.68) (size 0.6) (drill 0.3) (layers "F.Cu" "B.Cu") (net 23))
 (segment (start 112.0725 86.66) (end 112.0725 85.875) (width 0.508) (layer "B.Cu") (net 23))
 (segment (start 111.0525 87.68) (end 112.0725 86.66) (width 0.508) (layer "B.Cu") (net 23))
 (segment (start 110.18 87.68) (end 111.0525 87.68) (width 0.508) (layer "B.Cu") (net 23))
 (segment (start 112.0725 85.875) (end 110.9375 84.74) (width 0.508) (layer "B.Cu") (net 23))
 (segment (start 107.21707 72.44) (end 108.65 73.87293) (width 0.2) (layer "F.Cu") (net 6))
 (segment (start 108.65 73.87293) (end 108.65 74.68994) (width 0.2) (layer "F.Cu") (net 6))
 (segment (start 101.69 72.44) (end 107.21707 72.44) (width 0.2) (layer "F.Cu") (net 6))
 (segment (start 100.05 74.08) (end 101.69 72.44) (width 0.2) (layer "F.Cu") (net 6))
 (segment (start 104.0599 76.62) (end 104.84 75.8399) (width 0.2) (layer "F.Cu") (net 4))
 (segment (start 104.84 75.8399) (end 104.84 74.68994) (width 0.2) (layer "F.Cu") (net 4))
 (segment (start 100.05 76.62) (end 104.0599 76.62) (width 0.2) (layer "F.Cu") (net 4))
 (segment (start 98.661 75.231) (end 100.94193 75.231) (width 0.2) (layer "F.Cu") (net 7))
 (segment (start 107.38 73.88) (end 107.38 74.68994) (width 0.2) (layer "F.Cu") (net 7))
 (segment (start 106.93 73.43) (end 107.38 73.88) (width 0.2) (layer "F.Cu") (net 7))
 (segment (start 102.74293 73.43) (end 106.93 73.43) (width 0.2) (layer "F.Cu") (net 7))
 (segment (start 97.51 74.08) (end 98.661 75.231) (width 0.2) (layer "F.Cu") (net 7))
 (segment (start 100.94193 75.231) (end 102.74293 73.43) (width 0.2) (layer "F.Cu") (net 7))
 (segment (start 115.15695 79.16) (end 118.81 75.50695) (width 0.2) (layer "F.Cu") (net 3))
 (segment (start 100.05 79.16) (end 115.15695 79.16) (width 0.2) (layer "F.Cu") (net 3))
 (segment (start 118.81 75.50695) (end 118.81 74.68994) (width 0.2) (layer "F.Cu") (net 3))
 (segment (start 114.74796 82.54) (end 120.08 87.87204) (width 0.508) (layer "F.Cu") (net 2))
 (segment (start 120.08 87.87204) (end 120.08 89.33) (width 0.508) (layer "F.Cu") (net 2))
 (segment (start 99.5 81.15) (end 97.51 79.16) (width 0.508) (layer "F.Cu") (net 2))
 (segment (start 99.5 82.54) (end 114.74796 82.54) (width 0.508) (layer "F.Cu") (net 2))
 (segment (start 99.5 82.54) (end 99.5 81.15) (width 0.508) (layer "F.Cu") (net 2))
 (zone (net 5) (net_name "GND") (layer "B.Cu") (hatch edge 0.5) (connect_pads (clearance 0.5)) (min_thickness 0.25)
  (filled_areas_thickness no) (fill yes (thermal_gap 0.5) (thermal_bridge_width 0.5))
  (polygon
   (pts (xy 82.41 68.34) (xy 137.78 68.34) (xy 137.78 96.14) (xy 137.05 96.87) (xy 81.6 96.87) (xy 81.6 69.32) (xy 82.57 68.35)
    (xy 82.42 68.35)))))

